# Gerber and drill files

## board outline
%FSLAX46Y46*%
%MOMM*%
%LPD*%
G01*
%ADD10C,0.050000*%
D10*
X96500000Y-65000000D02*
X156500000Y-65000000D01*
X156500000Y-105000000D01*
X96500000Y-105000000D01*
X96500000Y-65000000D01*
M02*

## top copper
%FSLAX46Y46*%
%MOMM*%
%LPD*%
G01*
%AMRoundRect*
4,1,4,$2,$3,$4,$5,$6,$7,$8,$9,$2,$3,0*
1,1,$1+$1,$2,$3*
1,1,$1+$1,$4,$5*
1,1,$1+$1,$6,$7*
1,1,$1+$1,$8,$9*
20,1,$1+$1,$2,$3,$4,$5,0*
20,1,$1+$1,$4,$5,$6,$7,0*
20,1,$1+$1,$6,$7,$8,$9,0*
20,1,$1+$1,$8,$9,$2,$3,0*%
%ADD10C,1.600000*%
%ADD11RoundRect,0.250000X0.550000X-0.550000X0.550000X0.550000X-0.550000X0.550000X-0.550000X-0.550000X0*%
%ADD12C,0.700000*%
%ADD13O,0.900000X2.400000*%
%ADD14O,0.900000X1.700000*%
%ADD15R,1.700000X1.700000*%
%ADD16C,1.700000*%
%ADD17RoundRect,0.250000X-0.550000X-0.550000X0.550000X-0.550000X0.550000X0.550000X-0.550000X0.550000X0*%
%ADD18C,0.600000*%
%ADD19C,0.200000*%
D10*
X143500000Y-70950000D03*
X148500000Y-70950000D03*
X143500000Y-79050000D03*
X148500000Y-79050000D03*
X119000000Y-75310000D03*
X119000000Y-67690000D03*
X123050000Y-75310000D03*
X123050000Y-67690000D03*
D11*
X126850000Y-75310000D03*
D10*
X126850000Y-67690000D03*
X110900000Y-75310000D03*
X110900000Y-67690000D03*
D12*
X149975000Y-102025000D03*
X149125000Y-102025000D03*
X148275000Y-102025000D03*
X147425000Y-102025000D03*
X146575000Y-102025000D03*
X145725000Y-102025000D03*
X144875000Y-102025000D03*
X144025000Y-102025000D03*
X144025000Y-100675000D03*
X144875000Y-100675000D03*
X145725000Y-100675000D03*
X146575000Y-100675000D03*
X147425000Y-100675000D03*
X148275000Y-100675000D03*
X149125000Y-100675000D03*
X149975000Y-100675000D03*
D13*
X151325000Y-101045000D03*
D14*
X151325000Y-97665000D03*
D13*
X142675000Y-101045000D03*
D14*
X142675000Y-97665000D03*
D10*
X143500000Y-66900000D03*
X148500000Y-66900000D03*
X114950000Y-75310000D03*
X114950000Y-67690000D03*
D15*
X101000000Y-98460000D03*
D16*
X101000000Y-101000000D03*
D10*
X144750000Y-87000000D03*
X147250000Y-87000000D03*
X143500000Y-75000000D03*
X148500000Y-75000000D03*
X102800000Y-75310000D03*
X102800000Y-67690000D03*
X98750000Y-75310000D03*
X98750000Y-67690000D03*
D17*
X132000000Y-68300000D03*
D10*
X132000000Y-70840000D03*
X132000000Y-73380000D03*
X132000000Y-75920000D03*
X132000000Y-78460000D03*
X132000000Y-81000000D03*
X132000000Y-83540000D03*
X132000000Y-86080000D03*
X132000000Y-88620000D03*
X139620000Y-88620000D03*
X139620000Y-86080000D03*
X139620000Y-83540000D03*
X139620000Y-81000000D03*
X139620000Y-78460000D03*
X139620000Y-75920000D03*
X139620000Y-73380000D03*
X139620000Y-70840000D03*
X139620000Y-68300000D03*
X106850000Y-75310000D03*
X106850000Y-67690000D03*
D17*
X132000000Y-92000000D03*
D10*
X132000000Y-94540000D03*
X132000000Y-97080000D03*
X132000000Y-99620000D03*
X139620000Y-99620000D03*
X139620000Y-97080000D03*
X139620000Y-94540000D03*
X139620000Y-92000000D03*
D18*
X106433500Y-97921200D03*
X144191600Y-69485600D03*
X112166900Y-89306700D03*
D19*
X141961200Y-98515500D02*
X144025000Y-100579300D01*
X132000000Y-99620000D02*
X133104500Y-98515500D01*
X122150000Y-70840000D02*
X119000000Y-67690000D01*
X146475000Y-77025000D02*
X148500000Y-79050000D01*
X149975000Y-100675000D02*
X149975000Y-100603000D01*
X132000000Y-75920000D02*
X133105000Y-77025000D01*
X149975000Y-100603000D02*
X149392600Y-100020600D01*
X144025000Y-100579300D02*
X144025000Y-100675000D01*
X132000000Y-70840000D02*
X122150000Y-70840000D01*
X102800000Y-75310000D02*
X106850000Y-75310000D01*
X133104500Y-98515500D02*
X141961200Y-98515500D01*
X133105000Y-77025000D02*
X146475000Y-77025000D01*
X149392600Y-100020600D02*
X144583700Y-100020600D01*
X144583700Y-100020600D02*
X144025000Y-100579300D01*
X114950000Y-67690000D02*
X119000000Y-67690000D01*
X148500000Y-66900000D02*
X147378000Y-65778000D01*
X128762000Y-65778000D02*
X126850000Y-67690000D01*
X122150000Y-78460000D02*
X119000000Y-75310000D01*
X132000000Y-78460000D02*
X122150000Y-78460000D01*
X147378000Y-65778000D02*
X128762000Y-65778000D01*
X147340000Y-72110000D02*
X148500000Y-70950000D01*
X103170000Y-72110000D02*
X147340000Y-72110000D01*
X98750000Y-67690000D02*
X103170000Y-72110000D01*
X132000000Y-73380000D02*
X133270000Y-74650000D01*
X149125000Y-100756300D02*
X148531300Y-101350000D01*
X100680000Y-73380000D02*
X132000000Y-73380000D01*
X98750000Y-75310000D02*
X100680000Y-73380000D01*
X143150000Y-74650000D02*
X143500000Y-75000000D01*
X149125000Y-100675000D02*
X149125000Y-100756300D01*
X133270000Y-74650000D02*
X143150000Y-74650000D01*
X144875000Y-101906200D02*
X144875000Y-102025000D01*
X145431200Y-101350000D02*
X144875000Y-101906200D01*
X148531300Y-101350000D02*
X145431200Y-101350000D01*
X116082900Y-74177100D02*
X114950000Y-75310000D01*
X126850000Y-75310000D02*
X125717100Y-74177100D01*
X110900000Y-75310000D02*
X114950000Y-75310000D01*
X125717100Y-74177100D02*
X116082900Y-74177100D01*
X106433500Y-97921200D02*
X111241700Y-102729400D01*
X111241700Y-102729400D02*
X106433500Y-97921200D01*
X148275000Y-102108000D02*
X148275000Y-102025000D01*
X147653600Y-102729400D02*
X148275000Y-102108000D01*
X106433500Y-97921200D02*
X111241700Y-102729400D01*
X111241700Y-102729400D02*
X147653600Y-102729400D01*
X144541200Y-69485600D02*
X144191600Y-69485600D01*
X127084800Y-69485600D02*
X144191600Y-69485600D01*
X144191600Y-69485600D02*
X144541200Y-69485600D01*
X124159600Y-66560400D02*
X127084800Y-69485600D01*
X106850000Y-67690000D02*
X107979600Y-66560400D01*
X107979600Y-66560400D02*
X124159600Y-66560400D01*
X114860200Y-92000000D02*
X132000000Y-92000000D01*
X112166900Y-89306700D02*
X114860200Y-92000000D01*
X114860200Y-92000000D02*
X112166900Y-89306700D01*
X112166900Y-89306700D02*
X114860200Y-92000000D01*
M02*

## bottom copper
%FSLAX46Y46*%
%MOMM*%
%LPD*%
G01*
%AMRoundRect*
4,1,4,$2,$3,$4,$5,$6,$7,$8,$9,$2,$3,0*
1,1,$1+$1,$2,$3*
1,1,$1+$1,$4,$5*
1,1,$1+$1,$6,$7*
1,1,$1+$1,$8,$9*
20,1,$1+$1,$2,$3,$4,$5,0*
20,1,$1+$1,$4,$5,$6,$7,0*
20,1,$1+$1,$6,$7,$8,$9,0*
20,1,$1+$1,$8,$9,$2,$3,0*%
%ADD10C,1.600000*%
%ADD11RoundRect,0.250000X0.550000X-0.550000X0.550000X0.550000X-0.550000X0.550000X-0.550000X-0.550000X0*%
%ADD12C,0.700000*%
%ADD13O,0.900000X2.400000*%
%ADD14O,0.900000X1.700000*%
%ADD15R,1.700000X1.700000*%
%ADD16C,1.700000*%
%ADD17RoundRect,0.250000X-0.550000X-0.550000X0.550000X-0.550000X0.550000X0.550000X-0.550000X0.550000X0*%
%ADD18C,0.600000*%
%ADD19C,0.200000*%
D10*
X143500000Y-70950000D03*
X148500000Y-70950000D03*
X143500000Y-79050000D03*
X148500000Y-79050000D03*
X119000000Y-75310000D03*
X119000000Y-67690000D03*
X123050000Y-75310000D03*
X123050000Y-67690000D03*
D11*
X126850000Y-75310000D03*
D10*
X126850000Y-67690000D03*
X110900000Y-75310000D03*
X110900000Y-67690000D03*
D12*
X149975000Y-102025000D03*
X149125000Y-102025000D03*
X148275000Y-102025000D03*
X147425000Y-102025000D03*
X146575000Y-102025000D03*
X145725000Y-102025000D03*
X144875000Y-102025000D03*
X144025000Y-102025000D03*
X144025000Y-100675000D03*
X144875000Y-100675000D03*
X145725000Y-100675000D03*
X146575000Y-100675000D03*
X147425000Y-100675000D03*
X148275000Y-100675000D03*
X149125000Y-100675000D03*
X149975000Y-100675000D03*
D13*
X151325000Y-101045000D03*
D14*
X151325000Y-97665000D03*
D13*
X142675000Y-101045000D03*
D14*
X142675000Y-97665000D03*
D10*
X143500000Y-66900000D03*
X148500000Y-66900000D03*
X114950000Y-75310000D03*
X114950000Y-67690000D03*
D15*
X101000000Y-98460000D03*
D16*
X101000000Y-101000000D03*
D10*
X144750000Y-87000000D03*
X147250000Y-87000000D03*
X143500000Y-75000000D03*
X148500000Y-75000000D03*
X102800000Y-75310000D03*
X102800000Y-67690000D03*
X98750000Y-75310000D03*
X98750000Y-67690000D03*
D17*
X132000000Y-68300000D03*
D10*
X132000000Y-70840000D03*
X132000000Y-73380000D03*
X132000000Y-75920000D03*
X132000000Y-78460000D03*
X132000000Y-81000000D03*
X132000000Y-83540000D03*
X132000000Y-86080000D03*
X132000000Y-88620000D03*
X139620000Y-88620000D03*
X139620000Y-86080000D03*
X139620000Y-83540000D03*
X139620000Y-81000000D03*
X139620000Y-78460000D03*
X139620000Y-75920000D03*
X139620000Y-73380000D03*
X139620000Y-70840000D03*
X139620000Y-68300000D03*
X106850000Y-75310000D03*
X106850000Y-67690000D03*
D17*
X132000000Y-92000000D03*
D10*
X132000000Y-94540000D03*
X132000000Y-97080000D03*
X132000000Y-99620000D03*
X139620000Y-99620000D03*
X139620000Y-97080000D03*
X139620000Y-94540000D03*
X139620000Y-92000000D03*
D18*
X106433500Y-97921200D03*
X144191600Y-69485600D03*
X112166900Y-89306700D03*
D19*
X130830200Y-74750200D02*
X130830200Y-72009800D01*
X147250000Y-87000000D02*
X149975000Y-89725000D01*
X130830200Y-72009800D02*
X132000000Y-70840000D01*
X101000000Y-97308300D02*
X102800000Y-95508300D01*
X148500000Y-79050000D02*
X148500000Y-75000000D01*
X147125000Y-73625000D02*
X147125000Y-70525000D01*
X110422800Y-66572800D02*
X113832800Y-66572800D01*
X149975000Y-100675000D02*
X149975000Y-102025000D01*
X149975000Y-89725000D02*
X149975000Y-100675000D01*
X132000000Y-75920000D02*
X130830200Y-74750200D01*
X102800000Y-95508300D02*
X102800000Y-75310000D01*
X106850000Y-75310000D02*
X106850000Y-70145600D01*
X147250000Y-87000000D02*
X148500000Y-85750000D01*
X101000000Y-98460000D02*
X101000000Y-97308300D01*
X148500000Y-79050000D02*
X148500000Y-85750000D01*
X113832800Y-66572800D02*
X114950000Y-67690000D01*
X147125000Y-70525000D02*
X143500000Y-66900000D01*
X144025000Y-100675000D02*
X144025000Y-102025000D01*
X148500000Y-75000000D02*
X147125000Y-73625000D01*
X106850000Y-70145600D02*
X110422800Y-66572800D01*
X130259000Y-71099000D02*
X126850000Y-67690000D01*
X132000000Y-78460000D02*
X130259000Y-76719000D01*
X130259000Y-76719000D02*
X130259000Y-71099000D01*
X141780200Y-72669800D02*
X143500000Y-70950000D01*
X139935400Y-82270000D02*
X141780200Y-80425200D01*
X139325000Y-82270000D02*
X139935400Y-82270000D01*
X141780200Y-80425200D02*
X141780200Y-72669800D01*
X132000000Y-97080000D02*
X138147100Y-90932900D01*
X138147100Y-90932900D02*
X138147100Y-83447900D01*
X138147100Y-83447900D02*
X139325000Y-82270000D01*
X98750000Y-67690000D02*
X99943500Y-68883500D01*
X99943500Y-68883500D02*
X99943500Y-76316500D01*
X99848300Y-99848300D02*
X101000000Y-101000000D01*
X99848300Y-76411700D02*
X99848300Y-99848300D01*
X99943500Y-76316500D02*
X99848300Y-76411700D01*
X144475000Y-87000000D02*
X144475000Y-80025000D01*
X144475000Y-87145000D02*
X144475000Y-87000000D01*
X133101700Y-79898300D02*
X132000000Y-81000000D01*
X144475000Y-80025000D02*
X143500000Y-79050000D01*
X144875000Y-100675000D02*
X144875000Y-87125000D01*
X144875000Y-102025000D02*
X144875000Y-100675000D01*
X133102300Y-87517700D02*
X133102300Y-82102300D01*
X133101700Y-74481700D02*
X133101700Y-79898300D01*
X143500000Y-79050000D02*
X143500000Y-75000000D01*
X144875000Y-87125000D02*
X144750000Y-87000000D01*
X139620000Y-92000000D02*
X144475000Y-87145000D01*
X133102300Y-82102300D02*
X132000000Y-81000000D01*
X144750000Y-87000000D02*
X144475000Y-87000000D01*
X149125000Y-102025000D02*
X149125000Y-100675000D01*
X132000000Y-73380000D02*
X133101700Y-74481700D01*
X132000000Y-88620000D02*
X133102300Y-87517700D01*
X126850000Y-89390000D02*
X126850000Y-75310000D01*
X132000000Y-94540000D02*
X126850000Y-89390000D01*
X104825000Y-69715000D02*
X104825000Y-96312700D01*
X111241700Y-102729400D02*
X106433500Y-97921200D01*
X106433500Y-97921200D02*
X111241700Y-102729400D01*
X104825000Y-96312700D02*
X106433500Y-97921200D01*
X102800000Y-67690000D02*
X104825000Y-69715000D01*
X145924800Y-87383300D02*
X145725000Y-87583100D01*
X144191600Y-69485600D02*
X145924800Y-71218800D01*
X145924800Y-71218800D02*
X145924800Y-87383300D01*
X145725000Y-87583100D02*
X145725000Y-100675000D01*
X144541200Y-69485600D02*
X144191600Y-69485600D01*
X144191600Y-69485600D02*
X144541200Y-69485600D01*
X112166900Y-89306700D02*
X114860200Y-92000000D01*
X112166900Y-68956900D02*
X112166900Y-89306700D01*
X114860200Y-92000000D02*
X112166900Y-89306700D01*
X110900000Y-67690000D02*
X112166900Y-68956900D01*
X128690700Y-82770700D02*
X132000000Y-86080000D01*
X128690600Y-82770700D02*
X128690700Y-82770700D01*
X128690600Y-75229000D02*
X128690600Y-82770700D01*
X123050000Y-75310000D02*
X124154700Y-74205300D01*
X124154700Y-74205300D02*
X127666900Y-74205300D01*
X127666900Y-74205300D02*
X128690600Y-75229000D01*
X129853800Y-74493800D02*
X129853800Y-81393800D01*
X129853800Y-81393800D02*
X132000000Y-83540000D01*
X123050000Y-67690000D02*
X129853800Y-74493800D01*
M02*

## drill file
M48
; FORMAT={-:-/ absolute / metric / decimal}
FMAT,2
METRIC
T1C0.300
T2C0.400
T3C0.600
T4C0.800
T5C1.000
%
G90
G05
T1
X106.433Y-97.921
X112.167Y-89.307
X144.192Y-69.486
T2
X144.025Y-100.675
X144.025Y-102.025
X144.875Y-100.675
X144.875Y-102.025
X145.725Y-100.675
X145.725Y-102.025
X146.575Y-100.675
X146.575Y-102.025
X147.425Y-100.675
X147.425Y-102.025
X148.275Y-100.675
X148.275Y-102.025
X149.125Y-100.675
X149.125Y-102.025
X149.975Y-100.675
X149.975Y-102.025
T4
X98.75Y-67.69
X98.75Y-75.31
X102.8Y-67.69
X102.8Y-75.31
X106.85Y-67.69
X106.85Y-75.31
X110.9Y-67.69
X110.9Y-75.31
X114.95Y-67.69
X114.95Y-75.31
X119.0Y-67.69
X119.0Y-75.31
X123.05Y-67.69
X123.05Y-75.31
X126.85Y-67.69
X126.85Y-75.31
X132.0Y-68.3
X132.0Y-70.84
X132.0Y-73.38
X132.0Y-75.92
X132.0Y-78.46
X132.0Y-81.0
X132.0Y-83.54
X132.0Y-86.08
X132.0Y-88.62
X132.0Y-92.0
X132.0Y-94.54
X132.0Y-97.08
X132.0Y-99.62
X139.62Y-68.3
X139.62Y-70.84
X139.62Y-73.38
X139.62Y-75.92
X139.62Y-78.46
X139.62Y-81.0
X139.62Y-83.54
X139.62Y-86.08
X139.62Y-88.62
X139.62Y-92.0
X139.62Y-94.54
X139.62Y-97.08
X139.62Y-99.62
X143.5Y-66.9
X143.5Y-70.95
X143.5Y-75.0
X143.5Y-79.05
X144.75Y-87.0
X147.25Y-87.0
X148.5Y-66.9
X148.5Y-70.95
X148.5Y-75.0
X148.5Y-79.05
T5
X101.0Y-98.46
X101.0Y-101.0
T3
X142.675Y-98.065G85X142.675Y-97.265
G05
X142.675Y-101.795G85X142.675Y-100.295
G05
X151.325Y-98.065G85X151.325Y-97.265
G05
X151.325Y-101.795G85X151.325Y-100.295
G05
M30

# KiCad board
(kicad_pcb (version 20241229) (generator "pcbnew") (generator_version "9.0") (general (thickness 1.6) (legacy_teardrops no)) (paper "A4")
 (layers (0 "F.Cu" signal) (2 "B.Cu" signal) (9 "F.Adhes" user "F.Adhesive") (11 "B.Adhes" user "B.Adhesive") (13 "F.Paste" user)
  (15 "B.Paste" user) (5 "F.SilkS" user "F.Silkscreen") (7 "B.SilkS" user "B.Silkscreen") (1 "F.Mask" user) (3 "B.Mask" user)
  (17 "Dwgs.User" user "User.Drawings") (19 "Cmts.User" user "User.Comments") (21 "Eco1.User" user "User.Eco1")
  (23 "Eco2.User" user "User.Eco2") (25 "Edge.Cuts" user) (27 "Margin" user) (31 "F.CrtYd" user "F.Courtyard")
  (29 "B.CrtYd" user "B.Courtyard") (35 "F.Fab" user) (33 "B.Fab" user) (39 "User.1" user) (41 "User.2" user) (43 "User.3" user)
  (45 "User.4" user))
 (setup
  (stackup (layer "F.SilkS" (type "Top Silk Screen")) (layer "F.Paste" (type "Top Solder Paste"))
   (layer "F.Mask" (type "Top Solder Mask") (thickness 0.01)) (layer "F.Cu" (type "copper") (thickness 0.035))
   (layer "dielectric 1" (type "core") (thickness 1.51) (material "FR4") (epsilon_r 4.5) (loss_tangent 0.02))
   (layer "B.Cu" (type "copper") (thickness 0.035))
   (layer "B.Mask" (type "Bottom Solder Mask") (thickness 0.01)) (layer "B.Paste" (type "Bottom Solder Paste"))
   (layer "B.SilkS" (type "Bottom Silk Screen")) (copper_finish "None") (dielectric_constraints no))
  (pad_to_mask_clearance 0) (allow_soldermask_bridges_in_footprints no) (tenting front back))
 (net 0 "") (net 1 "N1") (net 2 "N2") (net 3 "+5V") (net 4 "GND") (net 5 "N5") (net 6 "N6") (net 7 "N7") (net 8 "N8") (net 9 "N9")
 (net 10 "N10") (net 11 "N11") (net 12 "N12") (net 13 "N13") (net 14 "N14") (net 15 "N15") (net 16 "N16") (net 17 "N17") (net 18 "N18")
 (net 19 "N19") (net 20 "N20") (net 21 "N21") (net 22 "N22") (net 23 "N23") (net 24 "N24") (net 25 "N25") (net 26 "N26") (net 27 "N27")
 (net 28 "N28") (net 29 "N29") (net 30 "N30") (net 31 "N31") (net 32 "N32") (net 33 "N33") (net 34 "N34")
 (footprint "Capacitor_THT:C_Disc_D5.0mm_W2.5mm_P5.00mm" (layer "F.Cu") (at 143.5 70.95)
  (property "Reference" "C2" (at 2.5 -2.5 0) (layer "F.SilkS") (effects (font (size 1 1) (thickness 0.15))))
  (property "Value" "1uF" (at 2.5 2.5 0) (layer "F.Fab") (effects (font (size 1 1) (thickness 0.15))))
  (pad "1" thru_hole circle (at 0 0) (size 1.6 1.6) (drill 0.8) (layers "*.Cu" "*.Mask") (remove_unused_layers no) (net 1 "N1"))
  (pad "2" thru_hole circle (at 5 0) (size 1.6 1.6) (drill 0.8) (layers "*.Cu" "*.Mask") (remove_unused_layers no) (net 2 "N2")))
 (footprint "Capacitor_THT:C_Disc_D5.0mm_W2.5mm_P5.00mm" (layer "F.Cu") (at 143.5 79.05)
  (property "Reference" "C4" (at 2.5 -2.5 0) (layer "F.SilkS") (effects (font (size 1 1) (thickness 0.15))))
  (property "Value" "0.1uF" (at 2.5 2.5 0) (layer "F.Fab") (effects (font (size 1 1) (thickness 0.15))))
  (pad "1" thru_hole circle (at 0 0) (size 1.6 1.6) (drill 0.8) (layers "*.Cu" "*.Mask") (remove_unused_layers no) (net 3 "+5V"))
  (pad "2" thru_hole circle (at 5 0) (size 1.6 1.6) (drill 0.8) (layers "*.Cu" "*.Mask") (remove_unused_layers no) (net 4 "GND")))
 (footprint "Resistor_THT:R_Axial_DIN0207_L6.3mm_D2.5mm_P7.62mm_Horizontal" (layer "F.Cu") (at 119 75.31 90)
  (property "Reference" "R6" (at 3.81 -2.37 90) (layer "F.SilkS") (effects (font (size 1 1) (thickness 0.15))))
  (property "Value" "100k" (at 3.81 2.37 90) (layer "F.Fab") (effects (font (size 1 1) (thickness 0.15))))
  (pad "1" thru_hole circle (at 0 0 90) (size 1.6 1.6) (drill 0.8) (layers "*.Cu" "*.Mask") (remove_unused_layers no) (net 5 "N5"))
  (pad "2" thru_hole circle (at 7.62 0 90) (size 1.6 1.6) (drill 0.8) (layers "*.Cu" "*.Mask") (remove_unused_layers no) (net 4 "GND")))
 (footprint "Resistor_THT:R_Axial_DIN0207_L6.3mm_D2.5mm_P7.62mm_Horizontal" (layer "F.Cu") (at 123.05 75.31 90)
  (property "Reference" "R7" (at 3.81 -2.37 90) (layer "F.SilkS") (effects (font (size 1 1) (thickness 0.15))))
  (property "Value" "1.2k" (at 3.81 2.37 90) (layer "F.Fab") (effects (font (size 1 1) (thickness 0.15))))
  (pad "1" thru_hole circle (at 0 0 90) (size 1.6 1.6) (drill 0.8) (layers "*.Cu" "*.Mask") (remove_unused_layers no) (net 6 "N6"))
  (pad "2" thru_hole circle (at 7.62 0 90) (size 1.6 1.6) (drill 0.8) (layers "*.Cu" "*.Mask") (remove_unused_layers no) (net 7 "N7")))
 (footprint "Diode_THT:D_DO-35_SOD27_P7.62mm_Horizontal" (layer "F.Cu") (at 126.85 75.31 90)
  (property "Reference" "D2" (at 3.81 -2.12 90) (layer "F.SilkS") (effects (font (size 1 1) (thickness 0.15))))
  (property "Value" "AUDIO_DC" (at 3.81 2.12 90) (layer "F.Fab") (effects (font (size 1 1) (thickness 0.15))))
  (pad "1" thru_hole roundrect (at 0 0 90) (size 1.6 1.6) (drill 0.8) (layers "*.Cu" "*.Mask") (remove_unused_layers no)
   (roundrect_rratio 0.15625) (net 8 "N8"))
  (pad "2" thru_hole circle (at 7.62 0 90) (size 1.6 1.6) (drill 0.8) (layers "*.Cu" "*.Mask") (remove_unused_layers no) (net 5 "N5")))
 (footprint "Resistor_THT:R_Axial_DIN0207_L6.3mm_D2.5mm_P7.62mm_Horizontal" (layer "F.Cu") (at 110.9 75.31 90)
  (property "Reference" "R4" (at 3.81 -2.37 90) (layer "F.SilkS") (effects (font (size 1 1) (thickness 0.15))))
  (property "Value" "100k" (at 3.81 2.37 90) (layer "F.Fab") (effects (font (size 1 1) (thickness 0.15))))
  (pad "1" thru_hole circle (at 0 0 90) (size 1.6 1.6) (drill 0.8) (layers "*.Cu" "*.Mask") (remove_unused_layers no) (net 8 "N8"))
  (pad "2" thru_hole circle (at 7.62 0 90) (size 1.6 1.6) (drill 0.8) (layers "*.Cu" "*.Mask") (remove_unused_layers no) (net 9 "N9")))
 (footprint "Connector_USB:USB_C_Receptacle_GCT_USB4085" (layer "F.Cu") (at 149.975 102.025 180)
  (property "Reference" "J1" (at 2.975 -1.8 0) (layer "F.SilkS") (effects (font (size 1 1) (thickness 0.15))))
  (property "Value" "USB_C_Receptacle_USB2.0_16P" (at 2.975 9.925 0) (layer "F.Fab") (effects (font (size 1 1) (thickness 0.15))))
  (pad "A1" thru_hole circle (at 0 0 180) (size 0.7 0.7) (drill 0.4) (layers "*.Cu" "*.Mask") (remove_unused_layers no) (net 4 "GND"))
  (pad "A4" thru_hole circle (at 0.85 0 180) (size 0.7 0.7) (drill 0.4) (layers "*.Cu" "*.Mask") (remove_unused_layers no) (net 3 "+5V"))
  (pad "A5" thru_hole circle (at 1.7 0 180) (size 0.7 0.7) (drill 0.4) (layers "*.Cu" "*.Mask") (remove_unused_layers no) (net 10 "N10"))
  (pad "A6" thru_hole circle (at 2.55 0 180) (size 0.7 0.7) (drill 0.4) (layers "*.Cu" "*.Mask") (remove_unused_layers no) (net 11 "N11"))
  (pad "A7" thru_hole circle (at 3.4 0 180) (size 0.7 0.7) (drill 0.4) (layers "*.Cu" "*.Mask") (remove_unused_layers no) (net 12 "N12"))
  (pad "A8" thru_hole circle (at 4.25 0 180) (size 0.7 0.7) (drill 0.4) (layers "*.Cu" "*.Mask") (remove_unused_layers no) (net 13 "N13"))
  (pad "A9" thru_hole circle (at 5.1 0 180) (size 0.7 0.7) (drill 0.4) (layers "*.Cu" "*.Mask") (remove_unused_layers no) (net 3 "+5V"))
  (pad "A12" thru_hole circle (at 5.95 0 180) (size 0.7 0.7) (drill 0.4) (layers "*.Cu" "*.Mask") (remove_unused_layers no) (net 4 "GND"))
  (pad "B1" thru_hole circle (at 5.95 1.35 180) (size 0.7 0.7) (drill 0.4) (layers "*.Cu" "*.Mask") (remove_unused_layers no) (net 4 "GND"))
  (pad "B4" thru_hole circle (at 5.1 1.35 180) (size 0.7 0.7) (drill 0.4) (layers "*.Cu" "*.Mask") (remove_unused_layers no) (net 3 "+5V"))
  (pad "B5" thru_hole circle (at 4.25 1.35 180) (size 0.7 0.7) (drill 0.4) (layers "*.Cu" "*.Mask") (remove_unused_layers no) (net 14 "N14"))
  (pad "B6" thru_hole circle (at 3.4 1.35 180) (size 0.7 0.7) (drill 0.4) (layers "*.Cu" "*.Mask") (remove_unused_layers no) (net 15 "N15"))
  (pad "B7" thru_hole circle (at 2.55 1.35 180) (size 0.7 0.7) (drill 0.4) (layers "*.Cu" "*.Mask") (remove_unused_layers no) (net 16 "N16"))
  (pad "B8" thru_hole circle (at 1.7 1.35 180) (size 0.7 0.7) (drill 0.4) (layers "*.Cu" "*.Mask") (remove_unused_layers no) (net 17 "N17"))
  (pad "B9" thru_hole circle (at 0.85 1.35 180) (size 0.7 0.7) (drill 0.4) (layers "*.Cu" "*.Mask") (remove_unused_layers no) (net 3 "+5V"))
  (pad "B12" thru_hole circle (at 0 1.35 180) (size 0.7 0.7) (drill 0.4) (layers "*.Cu" "*.Mask") (remove_unused_layers no) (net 4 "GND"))
  (pad "S1" thru_hole oval (at -1.35 0.98 180) (size 0.9 2.4) (drill oval 0.6 2.1) (layers "*.Cu" "*.Mask") (remove_unused_layers no)
   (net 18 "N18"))
  (pad "S1" thru_hole oval (at -1.35 4.36 180) (size 0.9 1.7) (drill oval 0.6 1.4) (layers "*.Cu" "*.Mask") (remove_unused_layers no)
   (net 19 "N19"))
  (pad "S1" thru_hole oval (at 7.3 0.98 180) (size 0.9 2.4) (drill oval 0.6 2.1) (layers "*.Cu" "*.Mask") (remove_unused_layers no)
   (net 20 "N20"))
  (pad "S1" thru_hole oval (at 7.3 4.36 180) (size 0.9 1.7) (drill oval 0.6 1.4) (layers "*.Cu" "*.Mask") (remove_unused_layers no)
   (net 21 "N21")))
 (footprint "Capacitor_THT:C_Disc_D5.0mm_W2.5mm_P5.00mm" (layer "F.Cu") (at 143.5 66.9)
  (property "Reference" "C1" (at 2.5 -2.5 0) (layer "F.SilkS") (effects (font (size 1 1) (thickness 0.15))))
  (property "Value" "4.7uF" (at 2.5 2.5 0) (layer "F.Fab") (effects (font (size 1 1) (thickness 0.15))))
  (pad "1" thru_hole circle (at 0 0) (size 1.6 1.6) (drill 0.8) (layers "*.Cu" "*.Mask") (remove_unused_layers no) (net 4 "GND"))
  (pad "2" thru_hole circle (at 5 0) (size 1.6 1.6) (drill 0.8) (layers "*.Cu" "*.Mask") (remove_unused_layers no) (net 5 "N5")))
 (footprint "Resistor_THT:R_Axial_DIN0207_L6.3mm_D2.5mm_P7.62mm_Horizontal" (layer "F.Cu") (at 114.95 75.31 90)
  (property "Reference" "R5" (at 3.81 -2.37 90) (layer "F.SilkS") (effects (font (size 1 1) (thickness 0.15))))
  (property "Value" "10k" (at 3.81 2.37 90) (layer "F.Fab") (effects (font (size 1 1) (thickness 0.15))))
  (pad "1" thru_hole circle (at 0 0 90) (size 1.6 1.6) (drill 0.8) (layers "*.Cu" "*.Mask") (remove_unused_layers no) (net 8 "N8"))
  (pad "2" thru_hole circle (at 7.62 0 90) (size 1.6 1.6) (drill 0.8) (layers "*.Cu" "*.Mask") (remove_unused_layers no) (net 4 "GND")))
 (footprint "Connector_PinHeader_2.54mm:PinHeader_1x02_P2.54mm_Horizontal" (layer "F.Cu") (at 101 98.46)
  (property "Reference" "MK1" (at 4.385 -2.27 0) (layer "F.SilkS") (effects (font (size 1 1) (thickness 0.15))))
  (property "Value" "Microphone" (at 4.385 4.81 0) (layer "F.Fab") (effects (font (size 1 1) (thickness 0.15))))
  (pad "1" thru_hole rect (at 0 0) (size 1.7 1.7) (drill 1) (layers "*.Cu" "*.Mask") (remove_unused_layers no) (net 4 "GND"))
  (pad "2" thru_hole circle (at 0 2.54) (size 1.7 1.7) (drill 1) (layers "*.Cu" "*.Mask") (remove_unused_layers no) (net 2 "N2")))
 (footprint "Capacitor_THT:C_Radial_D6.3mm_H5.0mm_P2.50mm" (layer "F.Cu") (at 144.75 87)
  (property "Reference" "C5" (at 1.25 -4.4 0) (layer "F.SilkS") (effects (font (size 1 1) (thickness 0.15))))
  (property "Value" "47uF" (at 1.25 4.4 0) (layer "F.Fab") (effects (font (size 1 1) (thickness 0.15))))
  (pad "1" thru_hole circle (at 0 0) (size 1.6 1.6) (drill 0.8) (layers "*.Cu" "*.Mask") (remove_unused_layers no) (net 3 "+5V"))
  (pad "2" thru_hole circle (at 2.5 0) (size 1.6 1.6) (drill 0.8) (layers "*.Cu" "*.Mask") (remove_unused_layers no) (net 4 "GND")))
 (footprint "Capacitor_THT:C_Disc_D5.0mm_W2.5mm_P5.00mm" (layer "F.Cu") (at 143.5 75)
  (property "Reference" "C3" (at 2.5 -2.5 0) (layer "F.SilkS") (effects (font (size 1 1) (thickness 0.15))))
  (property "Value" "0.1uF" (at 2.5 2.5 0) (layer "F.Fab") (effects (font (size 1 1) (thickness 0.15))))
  (pad "1" thru_hole circle (at 0 0) (size 1.6 1.6) (drill 0.8) (layers "*.Cu" "*.Mask") (remove_unused_layers no) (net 3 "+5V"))
  (pad "2" thru_hole circle (at 5 0) (size 1.6 1.6) (drill 0.8) (layers "*.Cu" "*.Mask") (remove_unused_layers no) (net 4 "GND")))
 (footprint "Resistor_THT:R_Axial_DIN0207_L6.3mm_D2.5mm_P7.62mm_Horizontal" (layer "F.Cu") (at 102.8 75.31 90)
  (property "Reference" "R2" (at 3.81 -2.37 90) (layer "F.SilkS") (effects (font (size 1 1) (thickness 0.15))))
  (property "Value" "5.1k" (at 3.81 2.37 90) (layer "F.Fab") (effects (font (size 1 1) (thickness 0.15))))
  (pad "1" thru_hole circle (at 0 0 90) (size 1.6 1.6) (drill 0.8) (layers "*.Cu" "*.Mask") (remove_unused_layers no) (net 4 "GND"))
  (pad "2" thru_hole circle (at 7.62 0 90) (size 1.6 1.6) (drill 0.8) (layers "*.Cu" "*.Mask") (remove_unused_layers no) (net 10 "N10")))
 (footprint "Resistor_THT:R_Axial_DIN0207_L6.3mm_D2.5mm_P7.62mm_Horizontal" (layer "F.Cu") (at 98.75 75.31 90)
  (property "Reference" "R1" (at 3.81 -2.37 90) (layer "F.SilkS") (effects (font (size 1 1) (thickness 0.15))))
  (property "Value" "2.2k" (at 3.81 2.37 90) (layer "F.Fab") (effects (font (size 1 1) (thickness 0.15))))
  (pad "1" thru_hole circle (at 0 0 90) (size 1.6 1.6) (drill 0.8) (layers "*.Cu" "*.Mask") (remove_unused_layers no) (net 3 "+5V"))
  (pad "2" thru_hole circle (at 7.62 0 90) (size 1.6 1.6) (drill 0.8) (layers "*.Cu" "*.Mask") (remove_unused_layers no) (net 2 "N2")))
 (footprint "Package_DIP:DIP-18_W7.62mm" (layer "F.Cu") (at 132 68.3)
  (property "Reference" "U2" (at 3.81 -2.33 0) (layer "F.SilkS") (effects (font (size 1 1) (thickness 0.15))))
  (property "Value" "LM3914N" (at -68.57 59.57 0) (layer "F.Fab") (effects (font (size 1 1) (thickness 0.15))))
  (pad "1" thru_hole roundrect (at 0 0) (size 1.6 1.6) (drill 0.8) (layers "*.Cu" "*.Mask") (remove_unused_layers no)
   (roundrect_rratio 0.15625) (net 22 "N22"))
  (pad "2" thru_hole circle (at 0 2.54) (size 1.6 1.6) (drill 0.8) (layers "*.Cu" "*.Mask") (remove_unused_layers no) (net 4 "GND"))
  (pad "3" thru_hole circle (at 0 5.08) (size 1.6 1.6) (drill 0.8) (layers "*.Cu" "*.Mask") (remove_unused_layers no) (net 3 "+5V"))
  (pad "4" thru_hole circle (at 0 7.62) (size 1.6 1.6) (drill 0.8) (layers "*.Cu" "*.Mask") (remove_unused_layers no) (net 4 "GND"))
  (pad "5" thru_hole circle (at 0 10.16) (size 1.6 1.6) (drill 0.8) (layers "*.Cu" "*.Mask") (remove_unused_layers no) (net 5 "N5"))
  (pad "6" thru_hole circle (at 0 12.7) (size 1.6 1.6) (drill 0.8) (layers "*.Cu" "*.Mask") (remove_unused_layers no) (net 3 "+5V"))
  (pad "7" thru_hole circle (at 0 15.24) (size 1.6 1.6) (drill 0.8) (layers "*.Cu" "*.Mask") (remove_unused_layers no) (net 7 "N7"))
  (pad "8" thru_hole circle (at 0 17.78) (size 1.6 1.6) (drill 0.8) (layers "*.Cu" "*.Mask") (remove_unused_layers no) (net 6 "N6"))
  (pad "9" thru_hole circle (at 0 20.32) (size 1.6 1.6) (drill 0.8) (layers "*.Cu" "*.Mask") (remove_unused_layers no) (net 3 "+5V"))
  (pad "10" thru_hole circle (at 7.62 20.32) (size 1.6 1.6) (drill 0.8) (layers "*.Cu" "*.Mask") (remove_unused_layers no) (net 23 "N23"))
  (pad "11" thru_hole circle (at 7.62 17.78) (size 1.6 1.6) (drill 0.8) (layers "*.Cu" "*.Mask") (remove_unused_layers no) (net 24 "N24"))
  (pad "12" thru_hole circle (at 7.62 15.24) (size 1.6 1.6) (drill 0.8) (layers "*.Cu" "*.Mask") (remove_unused_layers no) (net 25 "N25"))
  (pad "13" thru_hole circle (at 7.62 12.7) (size 1.6 1.6) (drill 0.8) (layers "*.Cu" "*.Mask") (remove_unused_layers no) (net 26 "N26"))
  (pad "14" thru_hole circle (at 7.62 10.16) (size 1.6 1.6) (drill 0.8) (layers "*.Cu" "*.Mask") (remove_unused_layers no) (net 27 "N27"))
  (pad "15" thru_hole circle (at 7.62 7.62) (size 1.6 1.6) (drill 0.8) (layers "*.Cu" "*.Mask") (remove_unused_layers no) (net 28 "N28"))
  (pad "16" thru_hole circle (at 7.62 5.08) (size 1.6 1.6) (drill 0.8) (layers "*.Cu" "*.Mask") (remove_unused_layers no) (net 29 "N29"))
  (pad "17" thru_hole circle (at 7.62 2.54) (size 1.6 1.6) (drill 0.8) (layers "*.Cu" "*.Mask") (remove_unused_layers no) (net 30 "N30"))
  (pad "18" thru_hole circle (at 7.62 0) (size 1.6 1.6) (drill 0.8) (layers "*.Cu" "*.Mask") (remove_unused_layers no) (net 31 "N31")))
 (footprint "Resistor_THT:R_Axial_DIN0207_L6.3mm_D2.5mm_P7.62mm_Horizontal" (layer "F.Cu") (at 106.85 75.31 90)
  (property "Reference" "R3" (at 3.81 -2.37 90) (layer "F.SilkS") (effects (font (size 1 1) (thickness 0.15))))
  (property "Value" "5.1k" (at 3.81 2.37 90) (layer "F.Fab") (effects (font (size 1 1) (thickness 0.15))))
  (pad "1" thru_hole circle (at 0 0 90) (size 1.6 1.6) (drill 0.8) (layers "*.Cu" "*.Mask") (remove_unused_layers no) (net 4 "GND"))
  (pad "2" thru_hole circle (at 7.62 0 90) (size 1.6 1.6) (drill 0.8) (layers "*.Cu" "*.Mask") (remove_unused_layers no) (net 14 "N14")))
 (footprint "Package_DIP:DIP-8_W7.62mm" (layer "F.Cu") (at 132 92)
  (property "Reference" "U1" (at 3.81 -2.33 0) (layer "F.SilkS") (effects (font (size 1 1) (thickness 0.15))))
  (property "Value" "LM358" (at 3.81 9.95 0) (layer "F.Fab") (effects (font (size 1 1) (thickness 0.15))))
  (pad "1" thru_hole roundrect (at 0 0) (size 1.6 1.6) (drill 0.8) (layers "*.Cu" "*.Mask") (remove_unused_layers no)
   (roundrect_rratio 0.15625) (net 9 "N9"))
  (pad "2" thru_hole circle (at 0 2.54) (size 1.6 1.6) (drill 0.8) (layers "*.Cu" "*.Mask") (remove_unused_layers no) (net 8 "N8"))
  (pad "3" thru_hole circle (at 0 5.08) (size 1.6 1.6) (drill 0.8) (layers "*.Cu" "*.Mask") (remove_unused_layers no) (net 1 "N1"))
  (pad "4" thru_hole circle (at 0 7.62) (size 1.6 1.6) (drill 0.8) (layers "*.Cu" "*.Mask") (remove_unused_layers no) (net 4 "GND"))
  (pad "5" thru_hole circle (at 7.62 7.62) (size 1.6 1.6) (drill 0.8) (layers "*.Cu" "*.Mask") (remove_unused_layers no) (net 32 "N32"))
  (pad "6" thru_hole circle (at 7.62 5.08) (size 1.6 1.6) (drill 0.8) (layers "*.Cu" "*.Mask") (remove_unused_layers no) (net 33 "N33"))
  (pad "7" thru_hole circle (at 7.62 2.54) (size 1.6 1.6) (drill 0.8) (layers "*.Cu" "*.Mask") (remove_unused_layers no) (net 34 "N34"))
  (pad "8" thru_hole circle (at 7.62 0) (size 1.6 1.6) (drill 0.8) (layers "*.Cu" "*.Mask") (remove_unused_layers no) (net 3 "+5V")))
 (gr_rect (start 96.5 65) (end 156.5 105) (stroke (width 0.05) (type default)) (fill no) (layer "Edge.Cuts"))
 (segment (start 141.9612 98.5155) (end 144.025 100.5793) (width 0.2) (layer "F.Cu") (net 4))
 (segment (start 132 99.62) (end 133.1045 98.5155) (width 0.2) (layer "F.Cu") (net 4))
 (segment (start 122.15 70.84) (end 119 67.69) (width 0.2) (layer "F.Cu") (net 4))
 (segment (start 146.475 77.025) (end 148.5 79.05) (width 0.2) (layer "F.Cu") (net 4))
 (segment (start 149.975 100.675) (end 149.975 100.603) (width 0.2) (layer "F.Cu") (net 4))
 (segment (start 132 75.92) (end 133.105 77.025) (width 0.2) (layer "F.Cu") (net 4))
 (segment (start 149.975 100.603) (end 149.3926 100.0206) (width 0.2) (layer "F.Cu") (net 4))
 (segment (start 144.025 100.5793) (end 144.025 100.675) (width 0.2) (layer "F.Cu") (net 4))
 (segment (start 132 70.84) (end 122.15 70.84) (width 0.2) (layer "F.Cu") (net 4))
 (segment (start 102.8 75.31) (end 106.85 75.31) (width 0.2) (layer "F.Cu") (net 4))
 (segment (start 133.1045 98.5155) (end 141.9612 98.5155) (width 0.2) (layer "F.Cu") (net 4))
 (segment (start 133.105 77.025) (end 146.475 77.025) (width 0.2) (layer "F.Cu") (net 4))
 (segment (start 149.3926 100.0206) (end 144.5837 100.0206) (width 0.2) (layer "F.Cu") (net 4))
 (segment (start 144.5837 100.0206) (end 144.025 100.5793) (width 0.2) (layer "F.Cu") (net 4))
 (segment (start 114.95 67.69) (end 119 67.69) (width 0.2) (layer "F.Cu") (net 4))
 (segment (start 130.8302 74.7502) (end 130.8302 72.0098) (width 0.2) (layer "B.Cu") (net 4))
 (segment (start 147.25 87) (end 149.975 89.725) (width 0.2) (layer "B.Cu") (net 4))
 (segment (start 130.8302 72.0098) (end 132 70.84) (width 0.2) (layer "B.Cu") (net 4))
 (segment (start 101 97.3083) (end 102.8 95.5083) (width 0.2) (layer "B.Cu") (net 4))
 (segment (start 148.5 79.05) (end 148.5 75) (width 0.2) (layer "B.Cu") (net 4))
 (segment (start 147.125 73.625) (end 147.125 70.525) (width 0.2) (layer "B.Cu") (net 4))
 (segment (start 110.4228 66.5728) (end 113.8328 66.5728) (width 0.2) (layer "B.Cu") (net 4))
 (segment (start 149.975 100.675) (end 149.975 102.025) (width 0.2) (layer "B.Cu") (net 4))
 (segment (start 149.975 89.725) (end 149.975 100.675) (width 0.2) (layer "B.Cu") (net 4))
 (segment (start 132 75.92) (end 130.8302 74.7502) (width 0.2) (layer "B.Cu") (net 4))
 (segment (start 102.8 95.5083) (end 102.8 75.31) (width 0.2) (layer "B.Cu") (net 4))
 (segment (start 106.85 75.31) (end 106.85 70.1456) (width 0.2) (layer "B.Cu") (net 4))
 (segment (start 147.25 87) (end 148.5 85.75) (width 0.2) (layer "B.Cu") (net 4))
 (segment (start 101 98.46) (end 101 97.3083) (width 0.2) (layer "B.Cu") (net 4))
 (segment (start 148.5 79.05) (end 148.5 85.75) (width 0.2) (layer "B.Cu") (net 4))
 (segment (start 113.8328 66.5728) (end 114.95 67.69) (width 0.2) (layer "B.Cu") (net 4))
 (segment (start 147.125 70.525) (end 143.5 66.9) (width 0.2) (layer "B.Cu") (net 4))
 (segment (start 144.025 100.675) (end 144.025 102.025) (width 0.2) (layer "B.Cu") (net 4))
 (segment (start 148.5 75) (end 147.125 73.625) (width 0.2) (layer "B.Cu") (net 4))
 (segment (start 106.85 70.1456) (end 110.4228 66.5728) (width 0.2) (layer "B.Cu") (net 4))
 (segment (start 148.5 66.9) (end 147.378 65.778) (width 0.2) (layer "F.Cu") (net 5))
 (segment (start 128.762 65.778) (end 126.85 67.69) (width 0.2) (layer "F.Cu") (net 5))
 (segment (start 122.15 78.46) (end 119 75.31) (width 0.2) (layer "F.Cu") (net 5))
 (segment (start 132 78.46) (end 122.15 78.46) (width 0.2) (layer "F.Cu") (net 5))
 (segment (start 147.378 65.778) (end 128.762 65.778) (width 0.2) (layer "F.Cu") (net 5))
 (segment (start 130.259 71.099) (end 126.85 67.69) (width 0.2) (layer "B.Cu") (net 5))
 (segment (start 132 78.46) (end 130.259 76.719) (width 0.2) (layer "B.Cu") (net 5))
 (segment (start 130.259 76.719) (end 130.259 71.099) (width 0.2) (layer "B.Cu") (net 5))
 (segment (start 141.7802 72.6698) (end 143.5 70.95) (width 0.2) (layer "B.Cu") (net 1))
 (segment (start 139.9354 82.27) (end 141.7802 80.4252) (width 0.2) (layer "B.Cu") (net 1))
 (segment (start 139.325 82.27) (end 139.9354 82.27) (width 0.2) (layer "B.Cu") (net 1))
 (segment (start 141.7802 80.4252) (end 141.7802 72.6698) (width 0.2) (layer "B.Cu") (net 1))
 (segment (start 132 97.08) (end 138.1471 90.9329) (width 0.2) (layer "B.Cu") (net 1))
 (segment (start 138.1471 90.9329) (end 138.1471 83.4479) (width 0.2) (layer "B.Cu") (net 1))
 (segment (start 138.1471 83.4479) (end 139.325 82.27) (width 0.2) (layer "B.Cu") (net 1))
 (segment (start 147.34 72.11) (end 148.5 70.95) (width 0.2) (layer "F.Cu") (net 2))
 (segment (start 103.17 72.11) (end 147.34 72.11) (width 0.2) (layer "F.Cu") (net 2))
 (segment (start 98.75 67.69) (end 103.17 72.11) (width 0.2) (layer "F.Cu") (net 2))
 (segment (start 98.75 67.69) (end 99.9435 68.8835) (width 0.2) (layer "B.Cu") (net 2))
 (segment (start 99.9435 68.8835) (end 99.9435 76.3165) (width 0.2) (layer "B.Cu") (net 2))
 (segment (start 99.8483 99.8483) (end 101 101) (width 0.2) (layer "B.Cu") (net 2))
 (segment (start 99.8483 76.4117) (end 99.8483 99.8483) (width 0.2) (layer "B.Cu") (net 2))
 (segment (start 99.9435 76.3165) (end 99.8483 76.4117) (width 0.2) (layer "B.Cu") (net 2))
 (segment (start 132 73.38) (end 133.27 74.65) (width 0.2) (layer "F.Cu") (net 3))
 (segment (start 149.125 100.7563) (end 148.5313 101.35) (width 0.2) (layer "F.Cu") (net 3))
 (segment (start 100.68 73.38) (end 132 73.38) (width 0.2) (layer "F.Cu") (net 3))
 (segment (start 98.75 75.31) (end 100.68 73.38) (width 0.2) (layer "F.Cu") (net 3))
 (segment (start 143.15 74.65) (end 143.5 75) (width 0.2) (layer "F.Cu") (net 3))
 (segment (start 149.125 100.675) (end 149.125 100.7563) (width 0.2) (layer "F.Cu") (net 3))
 (segment (start 133.27 74.65) (end 143.15 74.65) (width 0.2) (layer "F.Cu") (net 3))
 (segment (start 144.875 101.9062) (end 144.875 102.025) (width 0.2) (layer "F.Cu") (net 3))
 (segment (start 145.4312 101.35) (end 144.875 101.9062) (width 0.2) (layer "F.Cu") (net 3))
 (segment (start 148.5313 101.35) (end 145.4312 101.35) (width 0.2) (layer "F.Cu") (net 3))
 (segment (start 144.475 87) (end 144.475 80.025) (width 0.2) (layer "B.Cu") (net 3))
 (segment (start 144.475 87.145) (end 144.475 87) (width 0.2) (layer "B.Cu") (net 3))
 (segment (start 133.1017 79.8983) (end 132 81) (width 0.2) (layer "B.Cu") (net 3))
 (segment (start 144.475 80.025) (end 143.5 79.05) (width 0.2) (layer "B.Cu") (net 3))
 (segment (start 144.875 100.675) (end 144.875 87.125) (width 0.2) (layer "B.Cu") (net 3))
 (segment (start 144.875 102.025) (end 144.875 100.675) (width 0.2) (layer "B.Cu") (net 3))
 (segment (start 133.1023 87.5177) (end 133.1023 82.1023) (width 0.2) (layer "B.Cu") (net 3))
 (segment (start 133.1017 74.4817) (end 133.1017 79.8983) (width 0.2) (layer "B.Cu") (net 3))
 (segment (start 143.5 79.05) (end 143.5 75) (width 0.2) (layer "B.Cu") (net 3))
 (segment (start 144.875 87.125) (end 144.75 87) (width 0.2) (layer "B.Cu") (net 3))
 (segment (start 139.62 92) (end 144.475 87.145) (width 0.2) (layer "B.Cu") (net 3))
 (segment (start 133.1023 82.1023) (end 132 81) (width 0.2) (layer "B.Cu") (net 3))
 (segment (start 144.75 87) (end 144.475 87) (width 0.2) (layer "B.Cu") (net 3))
 (segment (start 149.125 102.025) (end 149.125 100.675) (width 0.2) (layer "B.Cu") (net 3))
 (segment (start 132 73.38) (end 133.1017 74.4817) (width 0.2) (layer "B.Cu") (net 3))
 (segment (start 132 88.62) (end 133.1023 87.5177) (width 0.2) (layer "B.Cu") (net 3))
 (segment (start 116.0829 74.1771) (end 114.95 75.31) (width 0.2) (layer "F.Cu") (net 8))
 (segment (start 126.85 75.31) (end 125.7171 74.1771) (width 0.2) (layer "F.Cu") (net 8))
 (segment (start 110.9 75.31) (end 114.95 75.31) (width 0.2) (layer "F.Cu") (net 8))
 (segment (start 125.7171 74.1771) (end 116.0829 74.1771) (width 0.2) (layer "F.Cu") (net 8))
 (segment (start 126.85 89.39) (end 126.85 75.31) (width 0.2) (layer "B.Cu") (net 8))
 (segment (start 132 94.54) (end 126.85 89.39) (width 0.2) (layer "B.Cu") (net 8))
 (segment (start 106.4335 97.9212) (end 111.2417 102.7294) (width 0.2) (layer "F.Cu") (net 10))
 (segment (start 111.2417 102.7294) (end 106.4335 97.9212) (width 0.2) (layer "F.Cu") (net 10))
 (segment (start 148.275 102.108) (end 148.275 102.025) (width 0.2) (layer "F.Cu") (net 10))
 (segment (start 147.6536 102.7294) (end 148.275 102.108) (width 0.2) (layer "F.Cu") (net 10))
 (segment (start 106.4335 97.9212) (end 111.2417 102.7294) (width 0.2) (layer "F.Cu") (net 10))
 (segment (start 111.2417 102.7294) (end 147.6536 102.7294) (width 0.2) (layer "F.Cu") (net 10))
 (via (at 106.4335 97.9212) (size 0.6) (drill 0.3) (layers "F.Cu" "B.Cu") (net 10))
 (segment (start 104.825 69.715) (end 104.825 96.3127) (width 0.2) (layer "B.Cu") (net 10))
 (segment (start 111.2417 102.7294) (end 106.4335 97.9212) (width 0.2) (layer "B.Cu") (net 10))
 (segment (start 106.4335 97.9212) (end 111.2417 102.7294) (width 0.2) (layer "B.Cu") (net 10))
 (segment (start 104.825 96.3127) (end 106.4335 97.9212) (width 0.2) (layer "B.Cu") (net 10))
 (segment (start 102.8 67.69) (end 104.825 69.715) (width 0.2) (layer "B.Cu") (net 10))
 (segment (start 144.5412 69.4856) (end 144.1916 69.4856) (width 0.2) (layer "F.Cu") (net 14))
 (segment (start 127.0848 69.4856) (end 144.1916 69.4856) (width 0.2) (layer "F.Cu") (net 14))
 (segment (start 144.1916 69.4856) (end 144.5412 69.4856) (width 0.2) (layer "F.Cu") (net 14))
 (segment (start 124.1596 66.5604) (end 127.0848 69.4856) (width 0.2) (layer "F.Cu") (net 14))
 (segment (start 106.85 67.69) (end 107.9796 66.5604) (width 0.2) (layer "F.Cu") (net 14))
 (segment (start 107.9796 66.5604) (end 124.1596 66.5604) (width 0.2) (layer "F.Cu") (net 14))
 (via (at 144.1916 69.4856) (size 0.6) (drill 0.3) (layers "F.Cu" "B.Cu") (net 14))
 (segment (start 145.9248 87.3833) (end 145.725 87.5831) (width 0.2) (layer "B.Cu") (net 14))
 (segment (start 144.1916 69.4856) (end 145.9248 71.2188) (width 0.2) (layer "B.Cu") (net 14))
 (segment (start 145.9248 71.2188) (end 145.9248 87.3833) (width 0.2) (layer "B.Cu") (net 14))
 (segment (start 145.725 87.5831) (end 145.725 100.675) (width 0.2) (layer "B.Cu") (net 14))
 (segment (start 144.5412 69.4856) (end 144.1916 69.4856) (width 0.2) (layer "B.Cu") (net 14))
 (segment (start 144.1916 69.4856) (end 144.5412 69.4856) (width 0.2) (layer "B.Cu") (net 14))
 (segment (start 114.8602 92) (end 132 92) (width 0.2) (layer "F.Cu") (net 9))
 (segment (start 112.1669 89.3067) (end 114.8602 92) (width 0.2) (layer "F.Cu") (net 9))
 (segment (start 114.8602 92) (end 112.1669 89.3067) (width 0.2) (layer "F.Cu") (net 9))
 (segment (start 112.1669 89.3067) (end 114.8602 92) (width 0.2) (layer "F.Cu") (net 9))
 (via (at 112.1669 89.3067) (size 0.6) (drill 0.3) (layers "F.Cu" "B.Cu") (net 9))
 (segment (start 112.1669 89.3067) (end 114.8602 92) (width 0.2) (layer "B.Cu") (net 9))
 (segment (start 112.1669 68.9569) (end 112.1669 89.3067) (width 0.2) (layer "B.Cu") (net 9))
 (segment (start 114.8602 92) (end 112.1669 89.3067) (width 0.2) (layer "B.Cu") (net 9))
 (segment (start 110.9 67.69) (end 112.1669 68.9569) (width 0.2) (layer "B.Cu") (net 9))
 (segment (start 128.6907 82.7707) (end 132 86.08) (width 0.2) (layer "B.Cu") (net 6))
 (segment (start 128.6906 82.7707) (end 128.6907 82.7707) (width 0.2) (layer "B.Cu") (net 6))
 (segment (start 128.6906 75.229) (end 128.6906 82.7707) (width 0.2) (layer "B.Cu") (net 6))
 (segment (start 123.05 75.31) (end 124.1547 74.2053) (width 0.2) (layer "B.Cu") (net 6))
 (segment (start 124.1547 74.2053) (end 127.6669 74.2053) (width 0.2) (layer "B.Cu") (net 6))
 (segment (start 127.6669 74.2053) (end 128.6906 75.229) (width 0.2) (layer "B.Cu") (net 6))
 (segment (start 129.8538 74.4938) (end 129.8538 81.3938) (width 0.2) (layer "B.Cu") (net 7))
 (segment (start 129.8538 81.3938) (end 132 83.54) (width 0.2) (layer "B.Cu") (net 7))
 (segment (start 123.05 67.69) (end 129.8538 74.4938) (width 0.2) (layer "B.Cu") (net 7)))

